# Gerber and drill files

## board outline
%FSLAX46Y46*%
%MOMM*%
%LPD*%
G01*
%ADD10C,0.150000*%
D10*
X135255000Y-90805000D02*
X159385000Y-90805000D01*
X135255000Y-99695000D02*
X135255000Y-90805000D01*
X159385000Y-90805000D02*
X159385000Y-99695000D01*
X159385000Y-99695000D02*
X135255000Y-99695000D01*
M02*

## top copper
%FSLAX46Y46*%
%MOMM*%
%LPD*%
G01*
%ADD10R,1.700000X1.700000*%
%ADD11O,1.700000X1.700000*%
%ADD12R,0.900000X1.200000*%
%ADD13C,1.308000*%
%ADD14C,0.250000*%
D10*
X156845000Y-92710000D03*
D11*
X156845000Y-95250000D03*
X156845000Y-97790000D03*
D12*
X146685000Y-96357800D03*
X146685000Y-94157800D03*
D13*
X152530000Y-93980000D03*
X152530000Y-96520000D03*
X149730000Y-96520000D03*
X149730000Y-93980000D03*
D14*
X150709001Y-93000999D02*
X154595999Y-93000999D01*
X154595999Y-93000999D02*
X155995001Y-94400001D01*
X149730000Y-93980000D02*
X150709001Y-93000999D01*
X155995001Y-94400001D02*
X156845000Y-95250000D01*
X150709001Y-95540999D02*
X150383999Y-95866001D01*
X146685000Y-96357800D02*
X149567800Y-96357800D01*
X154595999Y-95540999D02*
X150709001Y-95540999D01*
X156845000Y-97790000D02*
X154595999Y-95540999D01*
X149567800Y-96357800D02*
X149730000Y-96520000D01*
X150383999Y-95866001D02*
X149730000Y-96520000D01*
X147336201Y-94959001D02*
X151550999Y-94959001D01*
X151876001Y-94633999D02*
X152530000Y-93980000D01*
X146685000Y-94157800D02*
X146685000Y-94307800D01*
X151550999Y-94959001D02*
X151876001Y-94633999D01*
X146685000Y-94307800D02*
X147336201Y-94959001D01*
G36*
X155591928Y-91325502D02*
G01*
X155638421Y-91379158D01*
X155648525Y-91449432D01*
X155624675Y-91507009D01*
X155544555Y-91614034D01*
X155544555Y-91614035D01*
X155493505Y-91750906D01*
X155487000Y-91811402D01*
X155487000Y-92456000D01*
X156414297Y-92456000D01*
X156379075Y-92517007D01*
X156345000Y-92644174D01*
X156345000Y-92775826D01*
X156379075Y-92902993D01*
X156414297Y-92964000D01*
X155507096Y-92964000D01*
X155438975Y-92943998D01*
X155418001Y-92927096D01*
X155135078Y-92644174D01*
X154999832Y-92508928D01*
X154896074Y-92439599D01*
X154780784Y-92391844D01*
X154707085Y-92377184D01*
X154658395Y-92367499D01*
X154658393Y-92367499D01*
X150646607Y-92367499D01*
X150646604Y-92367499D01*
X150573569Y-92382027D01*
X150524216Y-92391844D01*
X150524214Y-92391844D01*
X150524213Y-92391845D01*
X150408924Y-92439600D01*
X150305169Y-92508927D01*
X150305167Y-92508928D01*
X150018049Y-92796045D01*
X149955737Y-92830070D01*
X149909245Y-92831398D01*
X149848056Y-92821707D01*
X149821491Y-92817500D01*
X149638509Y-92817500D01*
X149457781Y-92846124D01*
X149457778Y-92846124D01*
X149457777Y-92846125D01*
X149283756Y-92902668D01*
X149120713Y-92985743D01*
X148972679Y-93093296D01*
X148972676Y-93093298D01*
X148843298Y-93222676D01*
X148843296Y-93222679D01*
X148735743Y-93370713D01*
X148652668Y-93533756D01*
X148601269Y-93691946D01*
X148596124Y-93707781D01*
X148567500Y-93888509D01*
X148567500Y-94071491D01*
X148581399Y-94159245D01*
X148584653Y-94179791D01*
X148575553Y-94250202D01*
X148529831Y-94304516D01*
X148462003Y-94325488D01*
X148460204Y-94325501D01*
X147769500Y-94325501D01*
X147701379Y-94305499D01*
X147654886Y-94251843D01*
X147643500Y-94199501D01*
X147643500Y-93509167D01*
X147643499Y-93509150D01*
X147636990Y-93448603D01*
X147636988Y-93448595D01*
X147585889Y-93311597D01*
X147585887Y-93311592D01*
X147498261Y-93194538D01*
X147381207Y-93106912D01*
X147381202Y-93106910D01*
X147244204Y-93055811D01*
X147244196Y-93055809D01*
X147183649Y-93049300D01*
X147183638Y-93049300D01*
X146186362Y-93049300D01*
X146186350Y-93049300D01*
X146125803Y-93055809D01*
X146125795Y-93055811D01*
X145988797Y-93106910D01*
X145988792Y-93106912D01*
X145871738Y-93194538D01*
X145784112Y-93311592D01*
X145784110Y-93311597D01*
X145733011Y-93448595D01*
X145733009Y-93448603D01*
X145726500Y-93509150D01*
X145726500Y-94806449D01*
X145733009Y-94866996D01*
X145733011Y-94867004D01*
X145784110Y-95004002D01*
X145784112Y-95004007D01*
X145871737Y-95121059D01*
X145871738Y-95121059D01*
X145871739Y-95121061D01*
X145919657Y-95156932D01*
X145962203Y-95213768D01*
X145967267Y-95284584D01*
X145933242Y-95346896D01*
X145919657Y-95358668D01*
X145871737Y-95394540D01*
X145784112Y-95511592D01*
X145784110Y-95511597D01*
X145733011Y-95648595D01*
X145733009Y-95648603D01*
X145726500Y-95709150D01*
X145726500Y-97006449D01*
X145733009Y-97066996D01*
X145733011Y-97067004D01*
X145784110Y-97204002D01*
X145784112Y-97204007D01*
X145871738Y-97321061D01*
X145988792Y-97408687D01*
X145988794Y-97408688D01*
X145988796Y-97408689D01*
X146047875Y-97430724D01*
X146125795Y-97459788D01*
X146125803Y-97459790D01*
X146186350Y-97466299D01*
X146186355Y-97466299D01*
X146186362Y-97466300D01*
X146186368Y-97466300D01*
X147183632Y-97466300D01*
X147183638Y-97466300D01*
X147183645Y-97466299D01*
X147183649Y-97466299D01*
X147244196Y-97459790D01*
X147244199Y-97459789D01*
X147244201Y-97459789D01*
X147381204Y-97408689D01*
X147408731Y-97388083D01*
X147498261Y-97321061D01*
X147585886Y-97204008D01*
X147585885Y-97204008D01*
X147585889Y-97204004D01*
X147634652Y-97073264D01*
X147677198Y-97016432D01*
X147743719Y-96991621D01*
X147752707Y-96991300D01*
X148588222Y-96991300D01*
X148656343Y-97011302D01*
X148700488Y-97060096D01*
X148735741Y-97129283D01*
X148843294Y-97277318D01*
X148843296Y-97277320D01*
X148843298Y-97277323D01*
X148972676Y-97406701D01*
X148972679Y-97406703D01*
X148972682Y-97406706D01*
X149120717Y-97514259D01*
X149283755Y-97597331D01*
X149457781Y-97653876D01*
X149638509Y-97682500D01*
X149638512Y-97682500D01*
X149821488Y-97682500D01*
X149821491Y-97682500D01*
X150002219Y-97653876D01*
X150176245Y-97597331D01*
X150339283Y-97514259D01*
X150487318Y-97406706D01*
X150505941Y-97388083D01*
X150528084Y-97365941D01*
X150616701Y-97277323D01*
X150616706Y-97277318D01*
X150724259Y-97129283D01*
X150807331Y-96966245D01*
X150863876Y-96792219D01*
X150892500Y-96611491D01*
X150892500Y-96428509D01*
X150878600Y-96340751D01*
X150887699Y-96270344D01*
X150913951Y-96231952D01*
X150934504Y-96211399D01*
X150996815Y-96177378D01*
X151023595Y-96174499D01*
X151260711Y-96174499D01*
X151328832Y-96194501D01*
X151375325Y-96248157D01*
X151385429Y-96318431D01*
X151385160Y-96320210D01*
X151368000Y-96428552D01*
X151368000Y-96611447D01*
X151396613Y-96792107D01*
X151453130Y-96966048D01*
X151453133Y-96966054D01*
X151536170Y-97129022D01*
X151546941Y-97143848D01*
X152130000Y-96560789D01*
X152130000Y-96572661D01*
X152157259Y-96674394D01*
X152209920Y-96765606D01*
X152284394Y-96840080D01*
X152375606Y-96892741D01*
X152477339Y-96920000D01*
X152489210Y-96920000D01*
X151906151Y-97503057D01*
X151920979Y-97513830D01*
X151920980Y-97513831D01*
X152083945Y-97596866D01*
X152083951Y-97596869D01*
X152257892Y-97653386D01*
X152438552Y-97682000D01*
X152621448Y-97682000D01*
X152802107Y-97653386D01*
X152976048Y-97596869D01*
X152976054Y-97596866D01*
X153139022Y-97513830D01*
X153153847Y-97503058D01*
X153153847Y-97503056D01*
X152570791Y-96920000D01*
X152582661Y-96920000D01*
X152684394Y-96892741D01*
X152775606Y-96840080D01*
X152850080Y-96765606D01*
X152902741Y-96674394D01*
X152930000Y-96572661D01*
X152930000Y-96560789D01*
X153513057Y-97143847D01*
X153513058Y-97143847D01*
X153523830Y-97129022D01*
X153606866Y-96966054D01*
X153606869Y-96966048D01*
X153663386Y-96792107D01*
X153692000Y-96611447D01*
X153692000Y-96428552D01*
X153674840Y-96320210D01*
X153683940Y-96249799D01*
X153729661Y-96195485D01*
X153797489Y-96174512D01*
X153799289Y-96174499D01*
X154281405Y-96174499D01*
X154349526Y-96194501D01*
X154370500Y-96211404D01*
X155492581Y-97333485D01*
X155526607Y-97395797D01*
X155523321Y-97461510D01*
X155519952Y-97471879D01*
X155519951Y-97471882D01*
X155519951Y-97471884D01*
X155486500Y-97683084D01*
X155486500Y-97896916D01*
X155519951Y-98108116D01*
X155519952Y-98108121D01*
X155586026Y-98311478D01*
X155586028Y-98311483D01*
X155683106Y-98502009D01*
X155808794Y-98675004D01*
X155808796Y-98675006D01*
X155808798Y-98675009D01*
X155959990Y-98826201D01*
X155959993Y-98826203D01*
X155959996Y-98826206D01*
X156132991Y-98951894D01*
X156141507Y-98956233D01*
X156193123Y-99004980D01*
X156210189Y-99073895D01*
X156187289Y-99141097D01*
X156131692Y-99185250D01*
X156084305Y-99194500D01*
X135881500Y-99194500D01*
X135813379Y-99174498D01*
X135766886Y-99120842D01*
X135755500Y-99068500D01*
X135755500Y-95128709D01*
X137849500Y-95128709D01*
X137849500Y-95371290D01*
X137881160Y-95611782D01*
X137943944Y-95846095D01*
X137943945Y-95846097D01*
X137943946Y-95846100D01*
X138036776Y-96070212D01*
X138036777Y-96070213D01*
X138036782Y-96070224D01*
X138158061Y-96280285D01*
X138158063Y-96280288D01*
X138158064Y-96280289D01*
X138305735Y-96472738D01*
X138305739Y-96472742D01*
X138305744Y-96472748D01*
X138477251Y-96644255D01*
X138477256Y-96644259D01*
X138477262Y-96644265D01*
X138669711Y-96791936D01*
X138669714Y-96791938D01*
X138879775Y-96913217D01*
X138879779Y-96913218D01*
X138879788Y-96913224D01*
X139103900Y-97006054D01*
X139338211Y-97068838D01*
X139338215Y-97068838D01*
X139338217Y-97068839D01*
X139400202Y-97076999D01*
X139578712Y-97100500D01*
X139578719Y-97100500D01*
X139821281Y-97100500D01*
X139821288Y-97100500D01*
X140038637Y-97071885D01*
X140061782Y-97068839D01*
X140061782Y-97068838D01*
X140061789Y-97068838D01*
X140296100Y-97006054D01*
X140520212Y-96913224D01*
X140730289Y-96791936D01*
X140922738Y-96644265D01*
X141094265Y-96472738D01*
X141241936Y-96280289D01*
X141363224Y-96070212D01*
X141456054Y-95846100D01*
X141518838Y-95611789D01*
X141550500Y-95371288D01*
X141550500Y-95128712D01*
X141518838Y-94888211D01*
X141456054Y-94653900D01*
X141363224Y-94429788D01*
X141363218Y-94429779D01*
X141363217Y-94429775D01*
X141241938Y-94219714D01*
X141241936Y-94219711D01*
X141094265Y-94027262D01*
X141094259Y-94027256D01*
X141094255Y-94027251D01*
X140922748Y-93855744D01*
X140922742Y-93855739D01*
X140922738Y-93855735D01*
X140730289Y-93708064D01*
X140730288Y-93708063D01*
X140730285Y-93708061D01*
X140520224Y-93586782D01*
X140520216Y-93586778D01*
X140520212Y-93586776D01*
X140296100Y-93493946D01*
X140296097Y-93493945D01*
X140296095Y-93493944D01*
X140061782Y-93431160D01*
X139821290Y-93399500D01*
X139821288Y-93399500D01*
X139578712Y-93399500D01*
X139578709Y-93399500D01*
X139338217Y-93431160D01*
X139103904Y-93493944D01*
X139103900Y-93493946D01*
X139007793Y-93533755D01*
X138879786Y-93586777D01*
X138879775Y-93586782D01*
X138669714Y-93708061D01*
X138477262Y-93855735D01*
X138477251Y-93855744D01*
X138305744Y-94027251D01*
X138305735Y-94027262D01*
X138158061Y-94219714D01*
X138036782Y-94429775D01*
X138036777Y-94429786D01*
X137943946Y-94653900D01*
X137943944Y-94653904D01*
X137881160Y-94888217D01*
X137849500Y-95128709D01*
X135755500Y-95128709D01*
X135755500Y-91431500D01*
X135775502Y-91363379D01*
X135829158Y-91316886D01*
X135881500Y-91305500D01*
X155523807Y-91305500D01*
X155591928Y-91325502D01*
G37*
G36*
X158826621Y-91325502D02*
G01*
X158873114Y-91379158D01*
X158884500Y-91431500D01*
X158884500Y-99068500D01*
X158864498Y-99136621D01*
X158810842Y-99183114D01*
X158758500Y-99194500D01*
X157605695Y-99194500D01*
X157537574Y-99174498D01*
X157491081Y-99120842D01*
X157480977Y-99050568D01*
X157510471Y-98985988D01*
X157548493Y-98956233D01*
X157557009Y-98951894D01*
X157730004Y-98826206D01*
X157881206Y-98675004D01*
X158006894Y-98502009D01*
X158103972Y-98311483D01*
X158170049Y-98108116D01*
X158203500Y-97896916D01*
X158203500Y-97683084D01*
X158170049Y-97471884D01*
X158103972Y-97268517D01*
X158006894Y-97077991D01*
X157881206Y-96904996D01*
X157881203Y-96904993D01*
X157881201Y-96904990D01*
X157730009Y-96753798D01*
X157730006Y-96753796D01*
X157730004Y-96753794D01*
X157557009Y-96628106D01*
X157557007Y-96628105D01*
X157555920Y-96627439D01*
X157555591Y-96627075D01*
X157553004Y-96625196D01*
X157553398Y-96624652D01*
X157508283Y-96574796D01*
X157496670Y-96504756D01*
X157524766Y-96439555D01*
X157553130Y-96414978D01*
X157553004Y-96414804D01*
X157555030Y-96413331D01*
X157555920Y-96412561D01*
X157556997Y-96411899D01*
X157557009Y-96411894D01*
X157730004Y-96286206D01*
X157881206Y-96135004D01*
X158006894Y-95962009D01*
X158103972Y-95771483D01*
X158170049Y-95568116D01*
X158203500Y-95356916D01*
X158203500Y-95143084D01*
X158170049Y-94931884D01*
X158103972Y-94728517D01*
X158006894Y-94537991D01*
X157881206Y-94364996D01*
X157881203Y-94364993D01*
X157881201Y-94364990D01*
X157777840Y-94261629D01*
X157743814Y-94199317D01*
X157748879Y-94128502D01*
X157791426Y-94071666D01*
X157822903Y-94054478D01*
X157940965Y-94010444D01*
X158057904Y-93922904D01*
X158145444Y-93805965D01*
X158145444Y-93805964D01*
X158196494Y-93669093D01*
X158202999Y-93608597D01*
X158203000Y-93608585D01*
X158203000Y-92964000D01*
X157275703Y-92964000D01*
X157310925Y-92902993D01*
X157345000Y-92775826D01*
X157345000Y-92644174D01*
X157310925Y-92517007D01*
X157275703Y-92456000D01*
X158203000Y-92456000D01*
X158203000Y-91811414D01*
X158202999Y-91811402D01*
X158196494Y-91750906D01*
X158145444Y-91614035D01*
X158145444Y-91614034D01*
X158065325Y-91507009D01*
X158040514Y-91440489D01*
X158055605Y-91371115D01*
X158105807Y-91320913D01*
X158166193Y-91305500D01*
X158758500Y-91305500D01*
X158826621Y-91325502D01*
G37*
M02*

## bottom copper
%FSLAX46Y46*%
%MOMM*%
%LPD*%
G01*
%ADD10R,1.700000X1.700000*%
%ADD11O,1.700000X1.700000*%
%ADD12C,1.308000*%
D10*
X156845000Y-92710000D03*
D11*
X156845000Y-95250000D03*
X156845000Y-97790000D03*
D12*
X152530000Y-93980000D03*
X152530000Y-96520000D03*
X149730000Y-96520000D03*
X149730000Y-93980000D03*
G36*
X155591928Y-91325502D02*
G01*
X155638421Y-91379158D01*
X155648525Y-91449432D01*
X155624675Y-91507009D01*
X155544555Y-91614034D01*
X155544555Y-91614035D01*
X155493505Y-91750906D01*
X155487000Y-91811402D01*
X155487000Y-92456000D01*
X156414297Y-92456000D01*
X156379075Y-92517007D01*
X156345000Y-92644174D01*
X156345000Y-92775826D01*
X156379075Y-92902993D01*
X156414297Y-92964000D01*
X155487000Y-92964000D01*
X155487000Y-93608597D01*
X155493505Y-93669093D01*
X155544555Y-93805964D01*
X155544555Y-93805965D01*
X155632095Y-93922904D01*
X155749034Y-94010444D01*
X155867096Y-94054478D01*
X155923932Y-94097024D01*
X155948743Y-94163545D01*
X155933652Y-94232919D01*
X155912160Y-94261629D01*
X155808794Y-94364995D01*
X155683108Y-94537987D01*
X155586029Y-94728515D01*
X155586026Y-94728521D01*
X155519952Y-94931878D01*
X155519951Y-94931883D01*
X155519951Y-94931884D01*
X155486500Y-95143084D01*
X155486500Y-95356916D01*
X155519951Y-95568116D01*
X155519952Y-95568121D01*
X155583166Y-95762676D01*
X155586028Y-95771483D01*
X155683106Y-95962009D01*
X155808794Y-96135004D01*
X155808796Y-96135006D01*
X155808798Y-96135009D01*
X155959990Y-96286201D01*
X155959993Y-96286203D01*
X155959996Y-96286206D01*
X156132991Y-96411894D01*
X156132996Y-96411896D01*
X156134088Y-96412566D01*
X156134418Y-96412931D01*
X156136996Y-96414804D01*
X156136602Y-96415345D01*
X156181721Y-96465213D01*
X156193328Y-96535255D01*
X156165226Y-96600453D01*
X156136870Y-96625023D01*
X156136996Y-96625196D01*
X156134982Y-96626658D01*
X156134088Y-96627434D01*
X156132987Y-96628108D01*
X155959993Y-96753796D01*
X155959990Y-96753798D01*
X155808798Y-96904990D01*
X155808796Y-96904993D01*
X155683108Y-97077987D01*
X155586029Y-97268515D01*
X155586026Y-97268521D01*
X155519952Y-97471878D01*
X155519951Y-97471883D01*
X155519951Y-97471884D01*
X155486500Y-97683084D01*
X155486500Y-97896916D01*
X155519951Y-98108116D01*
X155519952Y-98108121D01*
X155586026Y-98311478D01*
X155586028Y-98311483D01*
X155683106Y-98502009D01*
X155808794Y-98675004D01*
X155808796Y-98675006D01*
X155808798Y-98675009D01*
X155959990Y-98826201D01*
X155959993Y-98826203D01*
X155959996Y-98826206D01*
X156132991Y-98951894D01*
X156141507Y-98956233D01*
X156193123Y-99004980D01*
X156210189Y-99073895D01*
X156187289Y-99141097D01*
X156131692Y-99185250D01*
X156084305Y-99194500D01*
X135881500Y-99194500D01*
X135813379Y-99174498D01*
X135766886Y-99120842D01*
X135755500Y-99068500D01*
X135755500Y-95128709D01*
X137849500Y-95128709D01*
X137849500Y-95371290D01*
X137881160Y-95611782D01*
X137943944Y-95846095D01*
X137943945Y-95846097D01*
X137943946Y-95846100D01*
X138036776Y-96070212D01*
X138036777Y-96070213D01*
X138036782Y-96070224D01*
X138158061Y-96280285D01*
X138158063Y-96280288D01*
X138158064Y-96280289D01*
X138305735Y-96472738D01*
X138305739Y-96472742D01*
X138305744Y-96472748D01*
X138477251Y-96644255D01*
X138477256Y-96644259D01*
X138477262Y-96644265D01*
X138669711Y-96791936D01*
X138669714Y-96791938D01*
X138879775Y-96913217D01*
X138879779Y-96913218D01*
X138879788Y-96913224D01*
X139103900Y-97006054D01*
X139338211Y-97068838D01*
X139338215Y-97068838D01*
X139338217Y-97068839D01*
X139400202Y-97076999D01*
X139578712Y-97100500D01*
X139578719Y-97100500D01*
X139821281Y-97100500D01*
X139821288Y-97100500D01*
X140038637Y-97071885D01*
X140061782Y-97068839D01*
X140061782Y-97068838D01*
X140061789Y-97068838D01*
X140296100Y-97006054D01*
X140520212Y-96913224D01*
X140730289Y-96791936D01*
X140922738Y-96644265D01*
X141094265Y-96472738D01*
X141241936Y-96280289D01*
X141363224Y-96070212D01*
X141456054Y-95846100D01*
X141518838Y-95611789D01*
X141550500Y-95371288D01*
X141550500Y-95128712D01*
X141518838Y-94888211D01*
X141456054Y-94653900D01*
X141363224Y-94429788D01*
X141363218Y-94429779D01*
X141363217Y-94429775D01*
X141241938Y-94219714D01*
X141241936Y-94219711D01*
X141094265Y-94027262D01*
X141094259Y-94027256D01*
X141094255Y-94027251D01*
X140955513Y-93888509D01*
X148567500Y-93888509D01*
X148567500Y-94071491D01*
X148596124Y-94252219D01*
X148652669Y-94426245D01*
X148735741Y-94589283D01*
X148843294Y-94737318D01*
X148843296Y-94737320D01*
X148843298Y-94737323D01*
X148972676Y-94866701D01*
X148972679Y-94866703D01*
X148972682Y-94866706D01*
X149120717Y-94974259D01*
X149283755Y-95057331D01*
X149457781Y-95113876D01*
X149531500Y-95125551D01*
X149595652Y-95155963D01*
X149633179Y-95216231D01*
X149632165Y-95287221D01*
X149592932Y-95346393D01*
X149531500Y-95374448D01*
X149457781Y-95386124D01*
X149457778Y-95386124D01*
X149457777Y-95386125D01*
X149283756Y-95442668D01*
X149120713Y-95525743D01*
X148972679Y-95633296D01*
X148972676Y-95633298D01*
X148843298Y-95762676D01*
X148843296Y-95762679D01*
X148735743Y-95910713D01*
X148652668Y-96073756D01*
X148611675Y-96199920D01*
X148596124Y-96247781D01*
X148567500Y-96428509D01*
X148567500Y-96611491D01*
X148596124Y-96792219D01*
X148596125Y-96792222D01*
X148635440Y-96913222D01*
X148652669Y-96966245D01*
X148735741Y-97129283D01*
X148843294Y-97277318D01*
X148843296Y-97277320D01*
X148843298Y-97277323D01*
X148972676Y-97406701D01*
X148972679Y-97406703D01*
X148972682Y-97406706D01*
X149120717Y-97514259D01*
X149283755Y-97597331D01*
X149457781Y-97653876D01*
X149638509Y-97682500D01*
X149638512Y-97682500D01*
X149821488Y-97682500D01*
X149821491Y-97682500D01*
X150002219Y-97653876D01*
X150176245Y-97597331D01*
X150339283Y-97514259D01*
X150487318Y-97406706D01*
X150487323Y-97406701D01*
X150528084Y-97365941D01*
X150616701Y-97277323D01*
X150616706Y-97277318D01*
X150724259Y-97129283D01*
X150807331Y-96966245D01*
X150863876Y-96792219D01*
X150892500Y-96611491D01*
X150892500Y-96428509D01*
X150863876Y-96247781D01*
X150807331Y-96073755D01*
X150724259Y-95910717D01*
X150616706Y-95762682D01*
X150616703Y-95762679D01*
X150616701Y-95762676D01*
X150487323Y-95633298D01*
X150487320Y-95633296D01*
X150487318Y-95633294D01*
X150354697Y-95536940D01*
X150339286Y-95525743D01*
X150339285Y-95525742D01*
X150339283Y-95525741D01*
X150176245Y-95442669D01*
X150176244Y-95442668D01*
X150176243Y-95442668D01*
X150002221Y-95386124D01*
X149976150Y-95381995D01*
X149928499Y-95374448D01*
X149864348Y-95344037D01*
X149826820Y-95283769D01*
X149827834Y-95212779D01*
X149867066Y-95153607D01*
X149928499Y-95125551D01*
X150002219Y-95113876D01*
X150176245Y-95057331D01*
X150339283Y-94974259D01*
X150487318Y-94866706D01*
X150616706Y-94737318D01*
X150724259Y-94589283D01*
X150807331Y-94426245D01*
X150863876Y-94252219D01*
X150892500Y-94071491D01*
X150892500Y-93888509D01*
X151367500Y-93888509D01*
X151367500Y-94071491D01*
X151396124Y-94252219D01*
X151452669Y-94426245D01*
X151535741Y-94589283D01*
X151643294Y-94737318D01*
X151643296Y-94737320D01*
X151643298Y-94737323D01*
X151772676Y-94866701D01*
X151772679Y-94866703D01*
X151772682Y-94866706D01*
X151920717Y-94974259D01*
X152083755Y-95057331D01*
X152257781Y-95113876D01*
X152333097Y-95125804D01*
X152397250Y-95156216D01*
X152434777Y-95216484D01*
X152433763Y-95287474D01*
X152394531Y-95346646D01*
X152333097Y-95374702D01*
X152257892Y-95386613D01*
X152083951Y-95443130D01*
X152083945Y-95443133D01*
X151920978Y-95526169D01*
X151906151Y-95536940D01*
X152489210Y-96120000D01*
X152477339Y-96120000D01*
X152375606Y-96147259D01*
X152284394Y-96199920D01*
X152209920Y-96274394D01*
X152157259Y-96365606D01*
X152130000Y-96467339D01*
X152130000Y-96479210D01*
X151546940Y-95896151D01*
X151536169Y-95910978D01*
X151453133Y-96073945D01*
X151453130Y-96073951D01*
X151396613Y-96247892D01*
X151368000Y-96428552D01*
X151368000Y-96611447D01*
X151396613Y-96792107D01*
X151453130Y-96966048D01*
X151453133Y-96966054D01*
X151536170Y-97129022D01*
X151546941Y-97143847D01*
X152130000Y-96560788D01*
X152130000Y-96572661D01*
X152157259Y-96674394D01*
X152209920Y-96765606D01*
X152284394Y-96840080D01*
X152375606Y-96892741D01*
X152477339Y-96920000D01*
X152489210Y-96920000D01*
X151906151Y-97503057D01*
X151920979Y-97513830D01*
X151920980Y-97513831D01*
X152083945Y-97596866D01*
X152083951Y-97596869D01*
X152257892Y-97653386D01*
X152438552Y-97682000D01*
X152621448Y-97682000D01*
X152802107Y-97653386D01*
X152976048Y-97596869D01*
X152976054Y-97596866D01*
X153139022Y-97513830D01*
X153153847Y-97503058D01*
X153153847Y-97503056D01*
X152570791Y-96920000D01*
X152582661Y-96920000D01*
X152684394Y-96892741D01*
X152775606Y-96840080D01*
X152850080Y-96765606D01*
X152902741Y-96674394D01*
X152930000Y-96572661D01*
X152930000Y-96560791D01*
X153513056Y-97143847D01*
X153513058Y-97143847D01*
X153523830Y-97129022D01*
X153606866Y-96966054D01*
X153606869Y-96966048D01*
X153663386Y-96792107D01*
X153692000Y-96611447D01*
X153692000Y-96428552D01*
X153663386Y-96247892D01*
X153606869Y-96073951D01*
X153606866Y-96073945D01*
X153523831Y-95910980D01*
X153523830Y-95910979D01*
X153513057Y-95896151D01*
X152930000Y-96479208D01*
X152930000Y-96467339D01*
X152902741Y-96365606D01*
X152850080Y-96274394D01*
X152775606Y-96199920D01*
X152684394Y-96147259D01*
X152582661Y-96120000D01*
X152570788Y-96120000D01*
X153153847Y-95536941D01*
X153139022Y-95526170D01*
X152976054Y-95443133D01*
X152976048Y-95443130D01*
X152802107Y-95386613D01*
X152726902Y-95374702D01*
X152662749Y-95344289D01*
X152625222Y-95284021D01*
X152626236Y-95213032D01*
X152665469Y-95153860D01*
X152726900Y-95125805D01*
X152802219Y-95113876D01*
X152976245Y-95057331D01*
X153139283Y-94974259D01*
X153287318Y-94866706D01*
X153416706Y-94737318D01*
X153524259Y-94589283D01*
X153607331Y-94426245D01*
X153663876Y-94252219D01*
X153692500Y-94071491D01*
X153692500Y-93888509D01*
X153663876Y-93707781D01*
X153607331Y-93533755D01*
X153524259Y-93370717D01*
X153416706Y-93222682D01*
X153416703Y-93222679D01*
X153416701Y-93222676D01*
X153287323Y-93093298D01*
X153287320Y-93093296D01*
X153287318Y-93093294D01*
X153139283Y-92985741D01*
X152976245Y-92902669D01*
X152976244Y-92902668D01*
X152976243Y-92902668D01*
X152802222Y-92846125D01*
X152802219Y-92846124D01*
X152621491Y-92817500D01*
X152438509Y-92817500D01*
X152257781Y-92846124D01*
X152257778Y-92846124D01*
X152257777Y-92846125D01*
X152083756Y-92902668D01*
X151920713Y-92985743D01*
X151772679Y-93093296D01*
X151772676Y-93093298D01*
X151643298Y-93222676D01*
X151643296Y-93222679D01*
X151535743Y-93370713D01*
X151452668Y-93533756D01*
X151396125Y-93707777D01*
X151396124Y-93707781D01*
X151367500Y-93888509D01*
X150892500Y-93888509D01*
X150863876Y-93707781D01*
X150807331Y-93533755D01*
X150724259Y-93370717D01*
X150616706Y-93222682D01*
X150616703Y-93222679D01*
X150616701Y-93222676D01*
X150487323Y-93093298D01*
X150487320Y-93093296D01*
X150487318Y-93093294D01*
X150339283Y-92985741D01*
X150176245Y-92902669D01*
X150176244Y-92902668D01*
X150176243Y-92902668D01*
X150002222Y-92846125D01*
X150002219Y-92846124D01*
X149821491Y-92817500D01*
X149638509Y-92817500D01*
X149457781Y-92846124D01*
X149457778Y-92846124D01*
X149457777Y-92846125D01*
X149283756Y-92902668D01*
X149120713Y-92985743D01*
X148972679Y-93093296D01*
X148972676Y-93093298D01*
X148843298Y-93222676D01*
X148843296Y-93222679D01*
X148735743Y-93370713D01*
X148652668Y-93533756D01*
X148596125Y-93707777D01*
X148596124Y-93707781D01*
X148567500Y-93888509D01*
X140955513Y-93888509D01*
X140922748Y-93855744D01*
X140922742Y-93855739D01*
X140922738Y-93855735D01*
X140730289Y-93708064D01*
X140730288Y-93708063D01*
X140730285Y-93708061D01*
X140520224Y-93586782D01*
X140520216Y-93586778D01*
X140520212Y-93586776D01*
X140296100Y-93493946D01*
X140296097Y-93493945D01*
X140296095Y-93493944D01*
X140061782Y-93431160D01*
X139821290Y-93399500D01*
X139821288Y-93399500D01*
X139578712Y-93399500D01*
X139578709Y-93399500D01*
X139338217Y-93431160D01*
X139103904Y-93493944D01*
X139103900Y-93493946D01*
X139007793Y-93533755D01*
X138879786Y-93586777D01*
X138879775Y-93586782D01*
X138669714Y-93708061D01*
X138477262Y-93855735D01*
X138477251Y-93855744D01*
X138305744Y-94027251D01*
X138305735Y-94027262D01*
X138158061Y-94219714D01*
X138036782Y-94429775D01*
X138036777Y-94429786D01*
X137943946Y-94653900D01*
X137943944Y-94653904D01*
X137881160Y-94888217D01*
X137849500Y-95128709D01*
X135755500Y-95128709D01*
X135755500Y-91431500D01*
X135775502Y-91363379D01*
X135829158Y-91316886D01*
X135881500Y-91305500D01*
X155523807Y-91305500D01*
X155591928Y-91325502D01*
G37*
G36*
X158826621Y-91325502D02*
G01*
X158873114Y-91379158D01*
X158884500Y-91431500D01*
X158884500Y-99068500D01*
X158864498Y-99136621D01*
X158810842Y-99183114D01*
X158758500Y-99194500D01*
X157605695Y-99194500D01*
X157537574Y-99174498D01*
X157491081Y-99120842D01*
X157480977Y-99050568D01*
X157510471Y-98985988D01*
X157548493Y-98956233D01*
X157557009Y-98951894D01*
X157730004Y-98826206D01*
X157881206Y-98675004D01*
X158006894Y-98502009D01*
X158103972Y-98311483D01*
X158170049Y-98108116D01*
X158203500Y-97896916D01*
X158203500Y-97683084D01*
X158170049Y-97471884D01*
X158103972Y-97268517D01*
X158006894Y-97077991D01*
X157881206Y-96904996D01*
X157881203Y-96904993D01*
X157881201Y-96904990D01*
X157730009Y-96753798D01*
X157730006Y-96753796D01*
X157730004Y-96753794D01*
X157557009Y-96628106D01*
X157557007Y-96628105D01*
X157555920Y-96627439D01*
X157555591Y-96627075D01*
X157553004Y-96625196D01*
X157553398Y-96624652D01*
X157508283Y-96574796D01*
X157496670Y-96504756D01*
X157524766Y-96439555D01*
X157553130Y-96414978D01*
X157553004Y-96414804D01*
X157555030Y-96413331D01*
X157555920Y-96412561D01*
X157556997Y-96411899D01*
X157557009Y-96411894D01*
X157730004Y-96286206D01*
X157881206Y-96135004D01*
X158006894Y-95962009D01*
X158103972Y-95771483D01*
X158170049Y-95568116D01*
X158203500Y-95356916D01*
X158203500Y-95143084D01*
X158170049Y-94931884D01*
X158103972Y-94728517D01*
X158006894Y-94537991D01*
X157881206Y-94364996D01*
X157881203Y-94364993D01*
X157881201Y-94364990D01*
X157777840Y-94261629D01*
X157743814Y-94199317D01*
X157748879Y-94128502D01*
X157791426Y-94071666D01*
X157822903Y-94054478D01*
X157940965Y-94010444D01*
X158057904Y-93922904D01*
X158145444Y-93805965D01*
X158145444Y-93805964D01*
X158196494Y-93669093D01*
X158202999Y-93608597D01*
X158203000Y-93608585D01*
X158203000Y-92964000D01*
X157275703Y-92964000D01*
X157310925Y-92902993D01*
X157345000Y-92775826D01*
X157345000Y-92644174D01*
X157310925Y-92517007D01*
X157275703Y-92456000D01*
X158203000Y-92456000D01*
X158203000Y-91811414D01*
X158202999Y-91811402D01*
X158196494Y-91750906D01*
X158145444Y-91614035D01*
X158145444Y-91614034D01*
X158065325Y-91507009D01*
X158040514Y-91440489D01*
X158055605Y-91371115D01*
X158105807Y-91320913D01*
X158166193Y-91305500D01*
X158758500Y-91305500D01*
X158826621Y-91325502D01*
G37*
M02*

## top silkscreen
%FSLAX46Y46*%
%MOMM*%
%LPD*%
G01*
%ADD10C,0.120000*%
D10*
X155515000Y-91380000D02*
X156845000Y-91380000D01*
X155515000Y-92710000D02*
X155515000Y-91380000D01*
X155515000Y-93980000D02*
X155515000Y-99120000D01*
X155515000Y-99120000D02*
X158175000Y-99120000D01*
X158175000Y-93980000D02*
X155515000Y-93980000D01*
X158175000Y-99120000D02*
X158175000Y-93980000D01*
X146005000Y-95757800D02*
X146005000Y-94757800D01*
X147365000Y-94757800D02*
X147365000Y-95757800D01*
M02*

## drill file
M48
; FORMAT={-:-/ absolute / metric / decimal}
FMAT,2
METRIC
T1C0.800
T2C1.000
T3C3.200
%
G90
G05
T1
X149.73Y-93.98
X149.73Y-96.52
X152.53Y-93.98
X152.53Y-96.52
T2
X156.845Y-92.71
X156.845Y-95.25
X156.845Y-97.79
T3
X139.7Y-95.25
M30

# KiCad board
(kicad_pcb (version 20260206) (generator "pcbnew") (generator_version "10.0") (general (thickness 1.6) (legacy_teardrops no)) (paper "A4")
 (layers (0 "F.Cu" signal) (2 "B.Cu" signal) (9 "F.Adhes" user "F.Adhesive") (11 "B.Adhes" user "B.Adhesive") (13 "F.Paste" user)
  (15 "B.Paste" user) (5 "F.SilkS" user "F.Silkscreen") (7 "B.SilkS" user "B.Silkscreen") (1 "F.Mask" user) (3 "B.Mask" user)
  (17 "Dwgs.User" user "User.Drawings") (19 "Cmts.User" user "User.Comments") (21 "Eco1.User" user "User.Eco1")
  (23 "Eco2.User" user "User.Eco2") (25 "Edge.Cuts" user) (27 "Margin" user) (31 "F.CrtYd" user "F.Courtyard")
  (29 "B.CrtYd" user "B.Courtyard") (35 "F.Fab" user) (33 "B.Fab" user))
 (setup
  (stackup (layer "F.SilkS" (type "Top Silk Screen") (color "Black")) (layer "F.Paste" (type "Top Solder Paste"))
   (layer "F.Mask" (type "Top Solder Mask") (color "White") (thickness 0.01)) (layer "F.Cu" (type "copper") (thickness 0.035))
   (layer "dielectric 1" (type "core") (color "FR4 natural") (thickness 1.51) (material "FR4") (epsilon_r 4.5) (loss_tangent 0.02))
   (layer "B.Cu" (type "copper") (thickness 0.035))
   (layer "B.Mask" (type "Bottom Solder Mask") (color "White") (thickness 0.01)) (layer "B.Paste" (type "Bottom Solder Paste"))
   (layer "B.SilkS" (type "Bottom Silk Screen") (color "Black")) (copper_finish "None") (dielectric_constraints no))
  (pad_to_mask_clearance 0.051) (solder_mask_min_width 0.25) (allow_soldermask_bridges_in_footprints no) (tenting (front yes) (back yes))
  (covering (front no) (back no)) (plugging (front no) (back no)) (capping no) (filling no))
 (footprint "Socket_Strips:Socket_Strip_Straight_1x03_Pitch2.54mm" (layer "F.Cu") (at 156.845 92.71)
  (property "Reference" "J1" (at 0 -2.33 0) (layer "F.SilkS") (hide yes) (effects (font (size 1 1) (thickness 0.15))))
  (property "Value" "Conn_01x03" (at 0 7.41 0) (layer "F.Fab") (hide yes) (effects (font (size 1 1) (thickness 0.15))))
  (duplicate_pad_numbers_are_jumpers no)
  (fp_line (start -1.33 -1.33) (end 0 -1.33) (stroke (width 0.12) (type solid)) (layer "F.SilkS"))
  (fp_line (start -1.33 0) (end -1.33 -1.33) (stroke (width 0.12) (type solid)) (layer "F.SilkS"))
  (fp_line (start -1.33 1.27) (end -1.33 6.41) (stroke (width 0.12) (type solid)) (layer "F.SilkS"))
  (fp_line (start -1.33 6.41) (end 1.33 6.41) (stroke (width 0.12) (type solid)) (layer "F.SilkS"))
  (fp_line (start 1.33 1.27) (end -1.33 1.27) (stroke (width 0.12) (type solid)) (layer "F.SilkS"))
  (fp_line (start 1.33 6.41) (end 1.33 1.27) (stroke (width 0.12) (type solid)) (layer "F.SilkS"))
  (pad "1" thru_hole rect (at 0 0) (size 1.7 1.7) (drill 1) (layers "*.Cu" "*.Mask") (remove_unused_layers no) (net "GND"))
  (pad "2" thru_hole oval (at 0 2.54) (size 1.7 1.7) (drill 1) (layers "*.Cu" "*.Mask") (remove_unused_layers no) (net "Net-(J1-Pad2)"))
  (pad "3" thru_hole oval (at 0 5.08) (size 1.7 1.7) (drill 1) (layers "*.Cu" "*.Mask") (remove_unused_layers no) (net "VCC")))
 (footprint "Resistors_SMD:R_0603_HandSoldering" (layer "F.Cu") (at 146.685 95.2578 90)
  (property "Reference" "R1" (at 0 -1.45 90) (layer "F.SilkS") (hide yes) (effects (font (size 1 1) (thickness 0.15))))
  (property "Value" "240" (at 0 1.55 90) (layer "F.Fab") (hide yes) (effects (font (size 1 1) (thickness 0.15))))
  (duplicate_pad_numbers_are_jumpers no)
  (fp_line (start -0.5 -0.68) (end 0.5 -0.68) (stroke (width 0.12) (type solid)) (layer "F.SilkS"))
  (fp_line (start 0.5 0.68) (end -0.5 0.68) (stroke (width 0.12) (type solid)) (layer "F.SilkS"))
  (pad "1" smd rect (at -1.1 0 90) (size 1.2 0.9) (layers "F.Cu" "F.Mask" "F.Paste") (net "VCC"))
  (pad "2" smd rect (at 1.1 0 90) (size 1.2 0.9) (layers "F.Cu" "F.Mask" "F.Paste") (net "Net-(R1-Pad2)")))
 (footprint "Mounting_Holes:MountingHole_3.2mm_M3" (layer "F.Cu") (at 139.7 95.25)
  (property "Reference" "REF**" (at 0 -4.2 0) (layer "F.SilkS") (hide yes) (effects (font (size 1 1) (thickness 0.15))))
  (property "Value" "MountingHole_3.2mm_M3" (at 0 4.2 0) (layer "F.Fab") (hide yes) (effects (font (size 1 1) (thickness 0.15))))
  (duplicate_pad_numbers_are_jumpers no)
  (pad "" np_thru_hole circle (at 0 0) (size 3.2 3.2) (drill 3.2) (layers "*.Cu" "*.Mask")))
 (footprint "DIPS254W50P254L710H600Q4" (layer "B.Cu") (at 151.13 95.25 180)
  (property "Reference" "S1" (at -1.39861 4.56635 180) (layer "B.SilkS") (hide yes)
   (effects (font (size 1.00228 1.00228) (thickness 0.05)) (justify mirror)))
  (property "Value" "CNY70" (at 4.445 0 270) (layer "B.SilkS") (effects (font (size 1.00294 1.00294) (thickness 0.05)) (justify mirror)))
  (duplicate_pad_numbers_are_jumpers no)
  (pad "A" thru_hole circle (at -1.4 1.27 180) (size 1.308 1.308) (drill 0.8) (layers "*.Cu" "*.Mask") (remove_unused_layers no)
   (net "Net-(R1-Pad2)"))
  (pad "CATH" thru_hole circle (at -1.4 -1.27 180) (size 1.308 1.308) (drill 0.8) (layers "*.Cu" "*.Mask") (remove_unused_layers no)
   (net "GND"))
  (pad "COLL" thru_hole circle (at 1.4 -1.27 180) (size 1.308 1.308) (drill 0.8) (layers "*.Cu" "*.Mask") (remove_unused_layers no)
   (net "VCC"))
  (pad "E" thru_hole circle (at 1.4 1.27 180) (size 1.308 1.308) (drill 0.8) (layers "*.Cu" "*.Mask") (remove_unused_layers no)
   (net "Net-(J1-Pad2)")))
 (gr_line (start 135.255 90.805) (end 159.385 90.805) (stroke (width 0.15) (type solid)) (layer "Edge.Cuts"))
 (gr_line (start 135.255 99.695) (end 135.255 90.805) (stroke (width 0.15) (type solid)) (layer "Edge.Cuts"))
 (gr_line (start 159.385 90.805) (end 159.385 99.695) (stroke (width 0.15) (type solid)) (layer "Edge.Cuts"))
 (gr_line (start 159.385 99.695) (end 135.255 99.695) (stroke (width 0.15) (type solid)) (layer "Edge.Cuts"))
 (segment (start 150.709001 93.000999) (end 154.595999 93.000999) (width 0.25) (layer "F.Cu") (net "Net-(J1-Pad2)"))
 (segment (start 154.595999 93.000999) (end 155.995001 94.400001) (width 0.25) (layer "F.Cu") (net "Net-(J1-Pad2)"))
 (segment (start 149.73 93.98) (end 150.709001 93.000999) (width 0.25) (layer "F.Cu") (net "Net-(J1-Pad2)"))
 (segment (start 155.995001 94.400001) (end 156.845 95.25) (width 0.25) (layer "F.Cu") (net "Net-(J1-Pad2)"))
 (segment (start 150.709001 95.540999) (end 150.383999 95.866001) (width 0.25) (layer "F.Cu") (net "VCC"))
 (segment (start 146.685 96.3578) (end 149.5678 96.3578) (width 0.25) (layer "F.Cu") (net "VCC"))
 (segment (start 154.595999 95.540999) (end 150.709001 95.540999) (width 0.25) (layer "F.Cu") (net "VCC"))
 (segment (start 156.845 97.79) (end 154.595999 95.540999) (width 0.25) (layer "F.Cu") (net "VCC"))
 (segment (start 149.5678 96.3578) (end 149.73 96.52) (width 0.25) (layer "F.Cu") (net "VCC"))
 (segment (start 150.383999 95.866001) (end 149.73 96.52) (width 0.25) (layer "F.Cu") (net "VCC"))
 (segment (start 147.336201 94.959001) (end 151.550999 94.959001) (width 0.25) (layer "F.Cu") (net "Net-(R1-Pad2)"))
 (segment (start 151.876001 94.633999) (end 152.53 93.98) (width 0.25) (layer "F.Cu") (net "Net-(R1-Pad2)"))
 (segment (start 146.685 94.1578) (end 146.685 94.3078) (width 0.25) (layer "F.Cu") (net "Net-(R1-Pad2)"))
 (segment (start 151.550999 94.959001) (end 151.876001 94.633999) (width 0.25) (layer "F.Cu") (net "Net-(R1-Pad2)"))
 (segment (start 146.685 94.3078) (end 147.336201 94.959001) (width 0.25) (layer "F.Cu") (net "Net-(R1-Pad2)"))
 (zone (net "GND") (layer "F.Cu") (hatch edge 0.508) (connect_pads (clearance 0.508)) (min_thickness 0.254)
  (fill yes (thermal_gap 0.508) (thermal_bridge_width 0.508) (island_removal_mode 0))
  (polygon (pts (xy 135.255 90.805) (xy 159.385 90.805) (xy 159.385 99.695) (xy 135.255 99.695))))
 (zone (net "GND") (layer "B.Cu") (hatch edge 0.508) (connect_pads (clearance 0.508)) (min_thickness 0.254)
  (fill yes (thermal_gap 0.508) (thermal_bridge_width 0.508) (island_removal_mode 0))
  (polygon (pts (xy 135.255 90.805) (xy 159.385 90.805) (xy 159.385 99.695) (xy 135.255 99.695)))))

